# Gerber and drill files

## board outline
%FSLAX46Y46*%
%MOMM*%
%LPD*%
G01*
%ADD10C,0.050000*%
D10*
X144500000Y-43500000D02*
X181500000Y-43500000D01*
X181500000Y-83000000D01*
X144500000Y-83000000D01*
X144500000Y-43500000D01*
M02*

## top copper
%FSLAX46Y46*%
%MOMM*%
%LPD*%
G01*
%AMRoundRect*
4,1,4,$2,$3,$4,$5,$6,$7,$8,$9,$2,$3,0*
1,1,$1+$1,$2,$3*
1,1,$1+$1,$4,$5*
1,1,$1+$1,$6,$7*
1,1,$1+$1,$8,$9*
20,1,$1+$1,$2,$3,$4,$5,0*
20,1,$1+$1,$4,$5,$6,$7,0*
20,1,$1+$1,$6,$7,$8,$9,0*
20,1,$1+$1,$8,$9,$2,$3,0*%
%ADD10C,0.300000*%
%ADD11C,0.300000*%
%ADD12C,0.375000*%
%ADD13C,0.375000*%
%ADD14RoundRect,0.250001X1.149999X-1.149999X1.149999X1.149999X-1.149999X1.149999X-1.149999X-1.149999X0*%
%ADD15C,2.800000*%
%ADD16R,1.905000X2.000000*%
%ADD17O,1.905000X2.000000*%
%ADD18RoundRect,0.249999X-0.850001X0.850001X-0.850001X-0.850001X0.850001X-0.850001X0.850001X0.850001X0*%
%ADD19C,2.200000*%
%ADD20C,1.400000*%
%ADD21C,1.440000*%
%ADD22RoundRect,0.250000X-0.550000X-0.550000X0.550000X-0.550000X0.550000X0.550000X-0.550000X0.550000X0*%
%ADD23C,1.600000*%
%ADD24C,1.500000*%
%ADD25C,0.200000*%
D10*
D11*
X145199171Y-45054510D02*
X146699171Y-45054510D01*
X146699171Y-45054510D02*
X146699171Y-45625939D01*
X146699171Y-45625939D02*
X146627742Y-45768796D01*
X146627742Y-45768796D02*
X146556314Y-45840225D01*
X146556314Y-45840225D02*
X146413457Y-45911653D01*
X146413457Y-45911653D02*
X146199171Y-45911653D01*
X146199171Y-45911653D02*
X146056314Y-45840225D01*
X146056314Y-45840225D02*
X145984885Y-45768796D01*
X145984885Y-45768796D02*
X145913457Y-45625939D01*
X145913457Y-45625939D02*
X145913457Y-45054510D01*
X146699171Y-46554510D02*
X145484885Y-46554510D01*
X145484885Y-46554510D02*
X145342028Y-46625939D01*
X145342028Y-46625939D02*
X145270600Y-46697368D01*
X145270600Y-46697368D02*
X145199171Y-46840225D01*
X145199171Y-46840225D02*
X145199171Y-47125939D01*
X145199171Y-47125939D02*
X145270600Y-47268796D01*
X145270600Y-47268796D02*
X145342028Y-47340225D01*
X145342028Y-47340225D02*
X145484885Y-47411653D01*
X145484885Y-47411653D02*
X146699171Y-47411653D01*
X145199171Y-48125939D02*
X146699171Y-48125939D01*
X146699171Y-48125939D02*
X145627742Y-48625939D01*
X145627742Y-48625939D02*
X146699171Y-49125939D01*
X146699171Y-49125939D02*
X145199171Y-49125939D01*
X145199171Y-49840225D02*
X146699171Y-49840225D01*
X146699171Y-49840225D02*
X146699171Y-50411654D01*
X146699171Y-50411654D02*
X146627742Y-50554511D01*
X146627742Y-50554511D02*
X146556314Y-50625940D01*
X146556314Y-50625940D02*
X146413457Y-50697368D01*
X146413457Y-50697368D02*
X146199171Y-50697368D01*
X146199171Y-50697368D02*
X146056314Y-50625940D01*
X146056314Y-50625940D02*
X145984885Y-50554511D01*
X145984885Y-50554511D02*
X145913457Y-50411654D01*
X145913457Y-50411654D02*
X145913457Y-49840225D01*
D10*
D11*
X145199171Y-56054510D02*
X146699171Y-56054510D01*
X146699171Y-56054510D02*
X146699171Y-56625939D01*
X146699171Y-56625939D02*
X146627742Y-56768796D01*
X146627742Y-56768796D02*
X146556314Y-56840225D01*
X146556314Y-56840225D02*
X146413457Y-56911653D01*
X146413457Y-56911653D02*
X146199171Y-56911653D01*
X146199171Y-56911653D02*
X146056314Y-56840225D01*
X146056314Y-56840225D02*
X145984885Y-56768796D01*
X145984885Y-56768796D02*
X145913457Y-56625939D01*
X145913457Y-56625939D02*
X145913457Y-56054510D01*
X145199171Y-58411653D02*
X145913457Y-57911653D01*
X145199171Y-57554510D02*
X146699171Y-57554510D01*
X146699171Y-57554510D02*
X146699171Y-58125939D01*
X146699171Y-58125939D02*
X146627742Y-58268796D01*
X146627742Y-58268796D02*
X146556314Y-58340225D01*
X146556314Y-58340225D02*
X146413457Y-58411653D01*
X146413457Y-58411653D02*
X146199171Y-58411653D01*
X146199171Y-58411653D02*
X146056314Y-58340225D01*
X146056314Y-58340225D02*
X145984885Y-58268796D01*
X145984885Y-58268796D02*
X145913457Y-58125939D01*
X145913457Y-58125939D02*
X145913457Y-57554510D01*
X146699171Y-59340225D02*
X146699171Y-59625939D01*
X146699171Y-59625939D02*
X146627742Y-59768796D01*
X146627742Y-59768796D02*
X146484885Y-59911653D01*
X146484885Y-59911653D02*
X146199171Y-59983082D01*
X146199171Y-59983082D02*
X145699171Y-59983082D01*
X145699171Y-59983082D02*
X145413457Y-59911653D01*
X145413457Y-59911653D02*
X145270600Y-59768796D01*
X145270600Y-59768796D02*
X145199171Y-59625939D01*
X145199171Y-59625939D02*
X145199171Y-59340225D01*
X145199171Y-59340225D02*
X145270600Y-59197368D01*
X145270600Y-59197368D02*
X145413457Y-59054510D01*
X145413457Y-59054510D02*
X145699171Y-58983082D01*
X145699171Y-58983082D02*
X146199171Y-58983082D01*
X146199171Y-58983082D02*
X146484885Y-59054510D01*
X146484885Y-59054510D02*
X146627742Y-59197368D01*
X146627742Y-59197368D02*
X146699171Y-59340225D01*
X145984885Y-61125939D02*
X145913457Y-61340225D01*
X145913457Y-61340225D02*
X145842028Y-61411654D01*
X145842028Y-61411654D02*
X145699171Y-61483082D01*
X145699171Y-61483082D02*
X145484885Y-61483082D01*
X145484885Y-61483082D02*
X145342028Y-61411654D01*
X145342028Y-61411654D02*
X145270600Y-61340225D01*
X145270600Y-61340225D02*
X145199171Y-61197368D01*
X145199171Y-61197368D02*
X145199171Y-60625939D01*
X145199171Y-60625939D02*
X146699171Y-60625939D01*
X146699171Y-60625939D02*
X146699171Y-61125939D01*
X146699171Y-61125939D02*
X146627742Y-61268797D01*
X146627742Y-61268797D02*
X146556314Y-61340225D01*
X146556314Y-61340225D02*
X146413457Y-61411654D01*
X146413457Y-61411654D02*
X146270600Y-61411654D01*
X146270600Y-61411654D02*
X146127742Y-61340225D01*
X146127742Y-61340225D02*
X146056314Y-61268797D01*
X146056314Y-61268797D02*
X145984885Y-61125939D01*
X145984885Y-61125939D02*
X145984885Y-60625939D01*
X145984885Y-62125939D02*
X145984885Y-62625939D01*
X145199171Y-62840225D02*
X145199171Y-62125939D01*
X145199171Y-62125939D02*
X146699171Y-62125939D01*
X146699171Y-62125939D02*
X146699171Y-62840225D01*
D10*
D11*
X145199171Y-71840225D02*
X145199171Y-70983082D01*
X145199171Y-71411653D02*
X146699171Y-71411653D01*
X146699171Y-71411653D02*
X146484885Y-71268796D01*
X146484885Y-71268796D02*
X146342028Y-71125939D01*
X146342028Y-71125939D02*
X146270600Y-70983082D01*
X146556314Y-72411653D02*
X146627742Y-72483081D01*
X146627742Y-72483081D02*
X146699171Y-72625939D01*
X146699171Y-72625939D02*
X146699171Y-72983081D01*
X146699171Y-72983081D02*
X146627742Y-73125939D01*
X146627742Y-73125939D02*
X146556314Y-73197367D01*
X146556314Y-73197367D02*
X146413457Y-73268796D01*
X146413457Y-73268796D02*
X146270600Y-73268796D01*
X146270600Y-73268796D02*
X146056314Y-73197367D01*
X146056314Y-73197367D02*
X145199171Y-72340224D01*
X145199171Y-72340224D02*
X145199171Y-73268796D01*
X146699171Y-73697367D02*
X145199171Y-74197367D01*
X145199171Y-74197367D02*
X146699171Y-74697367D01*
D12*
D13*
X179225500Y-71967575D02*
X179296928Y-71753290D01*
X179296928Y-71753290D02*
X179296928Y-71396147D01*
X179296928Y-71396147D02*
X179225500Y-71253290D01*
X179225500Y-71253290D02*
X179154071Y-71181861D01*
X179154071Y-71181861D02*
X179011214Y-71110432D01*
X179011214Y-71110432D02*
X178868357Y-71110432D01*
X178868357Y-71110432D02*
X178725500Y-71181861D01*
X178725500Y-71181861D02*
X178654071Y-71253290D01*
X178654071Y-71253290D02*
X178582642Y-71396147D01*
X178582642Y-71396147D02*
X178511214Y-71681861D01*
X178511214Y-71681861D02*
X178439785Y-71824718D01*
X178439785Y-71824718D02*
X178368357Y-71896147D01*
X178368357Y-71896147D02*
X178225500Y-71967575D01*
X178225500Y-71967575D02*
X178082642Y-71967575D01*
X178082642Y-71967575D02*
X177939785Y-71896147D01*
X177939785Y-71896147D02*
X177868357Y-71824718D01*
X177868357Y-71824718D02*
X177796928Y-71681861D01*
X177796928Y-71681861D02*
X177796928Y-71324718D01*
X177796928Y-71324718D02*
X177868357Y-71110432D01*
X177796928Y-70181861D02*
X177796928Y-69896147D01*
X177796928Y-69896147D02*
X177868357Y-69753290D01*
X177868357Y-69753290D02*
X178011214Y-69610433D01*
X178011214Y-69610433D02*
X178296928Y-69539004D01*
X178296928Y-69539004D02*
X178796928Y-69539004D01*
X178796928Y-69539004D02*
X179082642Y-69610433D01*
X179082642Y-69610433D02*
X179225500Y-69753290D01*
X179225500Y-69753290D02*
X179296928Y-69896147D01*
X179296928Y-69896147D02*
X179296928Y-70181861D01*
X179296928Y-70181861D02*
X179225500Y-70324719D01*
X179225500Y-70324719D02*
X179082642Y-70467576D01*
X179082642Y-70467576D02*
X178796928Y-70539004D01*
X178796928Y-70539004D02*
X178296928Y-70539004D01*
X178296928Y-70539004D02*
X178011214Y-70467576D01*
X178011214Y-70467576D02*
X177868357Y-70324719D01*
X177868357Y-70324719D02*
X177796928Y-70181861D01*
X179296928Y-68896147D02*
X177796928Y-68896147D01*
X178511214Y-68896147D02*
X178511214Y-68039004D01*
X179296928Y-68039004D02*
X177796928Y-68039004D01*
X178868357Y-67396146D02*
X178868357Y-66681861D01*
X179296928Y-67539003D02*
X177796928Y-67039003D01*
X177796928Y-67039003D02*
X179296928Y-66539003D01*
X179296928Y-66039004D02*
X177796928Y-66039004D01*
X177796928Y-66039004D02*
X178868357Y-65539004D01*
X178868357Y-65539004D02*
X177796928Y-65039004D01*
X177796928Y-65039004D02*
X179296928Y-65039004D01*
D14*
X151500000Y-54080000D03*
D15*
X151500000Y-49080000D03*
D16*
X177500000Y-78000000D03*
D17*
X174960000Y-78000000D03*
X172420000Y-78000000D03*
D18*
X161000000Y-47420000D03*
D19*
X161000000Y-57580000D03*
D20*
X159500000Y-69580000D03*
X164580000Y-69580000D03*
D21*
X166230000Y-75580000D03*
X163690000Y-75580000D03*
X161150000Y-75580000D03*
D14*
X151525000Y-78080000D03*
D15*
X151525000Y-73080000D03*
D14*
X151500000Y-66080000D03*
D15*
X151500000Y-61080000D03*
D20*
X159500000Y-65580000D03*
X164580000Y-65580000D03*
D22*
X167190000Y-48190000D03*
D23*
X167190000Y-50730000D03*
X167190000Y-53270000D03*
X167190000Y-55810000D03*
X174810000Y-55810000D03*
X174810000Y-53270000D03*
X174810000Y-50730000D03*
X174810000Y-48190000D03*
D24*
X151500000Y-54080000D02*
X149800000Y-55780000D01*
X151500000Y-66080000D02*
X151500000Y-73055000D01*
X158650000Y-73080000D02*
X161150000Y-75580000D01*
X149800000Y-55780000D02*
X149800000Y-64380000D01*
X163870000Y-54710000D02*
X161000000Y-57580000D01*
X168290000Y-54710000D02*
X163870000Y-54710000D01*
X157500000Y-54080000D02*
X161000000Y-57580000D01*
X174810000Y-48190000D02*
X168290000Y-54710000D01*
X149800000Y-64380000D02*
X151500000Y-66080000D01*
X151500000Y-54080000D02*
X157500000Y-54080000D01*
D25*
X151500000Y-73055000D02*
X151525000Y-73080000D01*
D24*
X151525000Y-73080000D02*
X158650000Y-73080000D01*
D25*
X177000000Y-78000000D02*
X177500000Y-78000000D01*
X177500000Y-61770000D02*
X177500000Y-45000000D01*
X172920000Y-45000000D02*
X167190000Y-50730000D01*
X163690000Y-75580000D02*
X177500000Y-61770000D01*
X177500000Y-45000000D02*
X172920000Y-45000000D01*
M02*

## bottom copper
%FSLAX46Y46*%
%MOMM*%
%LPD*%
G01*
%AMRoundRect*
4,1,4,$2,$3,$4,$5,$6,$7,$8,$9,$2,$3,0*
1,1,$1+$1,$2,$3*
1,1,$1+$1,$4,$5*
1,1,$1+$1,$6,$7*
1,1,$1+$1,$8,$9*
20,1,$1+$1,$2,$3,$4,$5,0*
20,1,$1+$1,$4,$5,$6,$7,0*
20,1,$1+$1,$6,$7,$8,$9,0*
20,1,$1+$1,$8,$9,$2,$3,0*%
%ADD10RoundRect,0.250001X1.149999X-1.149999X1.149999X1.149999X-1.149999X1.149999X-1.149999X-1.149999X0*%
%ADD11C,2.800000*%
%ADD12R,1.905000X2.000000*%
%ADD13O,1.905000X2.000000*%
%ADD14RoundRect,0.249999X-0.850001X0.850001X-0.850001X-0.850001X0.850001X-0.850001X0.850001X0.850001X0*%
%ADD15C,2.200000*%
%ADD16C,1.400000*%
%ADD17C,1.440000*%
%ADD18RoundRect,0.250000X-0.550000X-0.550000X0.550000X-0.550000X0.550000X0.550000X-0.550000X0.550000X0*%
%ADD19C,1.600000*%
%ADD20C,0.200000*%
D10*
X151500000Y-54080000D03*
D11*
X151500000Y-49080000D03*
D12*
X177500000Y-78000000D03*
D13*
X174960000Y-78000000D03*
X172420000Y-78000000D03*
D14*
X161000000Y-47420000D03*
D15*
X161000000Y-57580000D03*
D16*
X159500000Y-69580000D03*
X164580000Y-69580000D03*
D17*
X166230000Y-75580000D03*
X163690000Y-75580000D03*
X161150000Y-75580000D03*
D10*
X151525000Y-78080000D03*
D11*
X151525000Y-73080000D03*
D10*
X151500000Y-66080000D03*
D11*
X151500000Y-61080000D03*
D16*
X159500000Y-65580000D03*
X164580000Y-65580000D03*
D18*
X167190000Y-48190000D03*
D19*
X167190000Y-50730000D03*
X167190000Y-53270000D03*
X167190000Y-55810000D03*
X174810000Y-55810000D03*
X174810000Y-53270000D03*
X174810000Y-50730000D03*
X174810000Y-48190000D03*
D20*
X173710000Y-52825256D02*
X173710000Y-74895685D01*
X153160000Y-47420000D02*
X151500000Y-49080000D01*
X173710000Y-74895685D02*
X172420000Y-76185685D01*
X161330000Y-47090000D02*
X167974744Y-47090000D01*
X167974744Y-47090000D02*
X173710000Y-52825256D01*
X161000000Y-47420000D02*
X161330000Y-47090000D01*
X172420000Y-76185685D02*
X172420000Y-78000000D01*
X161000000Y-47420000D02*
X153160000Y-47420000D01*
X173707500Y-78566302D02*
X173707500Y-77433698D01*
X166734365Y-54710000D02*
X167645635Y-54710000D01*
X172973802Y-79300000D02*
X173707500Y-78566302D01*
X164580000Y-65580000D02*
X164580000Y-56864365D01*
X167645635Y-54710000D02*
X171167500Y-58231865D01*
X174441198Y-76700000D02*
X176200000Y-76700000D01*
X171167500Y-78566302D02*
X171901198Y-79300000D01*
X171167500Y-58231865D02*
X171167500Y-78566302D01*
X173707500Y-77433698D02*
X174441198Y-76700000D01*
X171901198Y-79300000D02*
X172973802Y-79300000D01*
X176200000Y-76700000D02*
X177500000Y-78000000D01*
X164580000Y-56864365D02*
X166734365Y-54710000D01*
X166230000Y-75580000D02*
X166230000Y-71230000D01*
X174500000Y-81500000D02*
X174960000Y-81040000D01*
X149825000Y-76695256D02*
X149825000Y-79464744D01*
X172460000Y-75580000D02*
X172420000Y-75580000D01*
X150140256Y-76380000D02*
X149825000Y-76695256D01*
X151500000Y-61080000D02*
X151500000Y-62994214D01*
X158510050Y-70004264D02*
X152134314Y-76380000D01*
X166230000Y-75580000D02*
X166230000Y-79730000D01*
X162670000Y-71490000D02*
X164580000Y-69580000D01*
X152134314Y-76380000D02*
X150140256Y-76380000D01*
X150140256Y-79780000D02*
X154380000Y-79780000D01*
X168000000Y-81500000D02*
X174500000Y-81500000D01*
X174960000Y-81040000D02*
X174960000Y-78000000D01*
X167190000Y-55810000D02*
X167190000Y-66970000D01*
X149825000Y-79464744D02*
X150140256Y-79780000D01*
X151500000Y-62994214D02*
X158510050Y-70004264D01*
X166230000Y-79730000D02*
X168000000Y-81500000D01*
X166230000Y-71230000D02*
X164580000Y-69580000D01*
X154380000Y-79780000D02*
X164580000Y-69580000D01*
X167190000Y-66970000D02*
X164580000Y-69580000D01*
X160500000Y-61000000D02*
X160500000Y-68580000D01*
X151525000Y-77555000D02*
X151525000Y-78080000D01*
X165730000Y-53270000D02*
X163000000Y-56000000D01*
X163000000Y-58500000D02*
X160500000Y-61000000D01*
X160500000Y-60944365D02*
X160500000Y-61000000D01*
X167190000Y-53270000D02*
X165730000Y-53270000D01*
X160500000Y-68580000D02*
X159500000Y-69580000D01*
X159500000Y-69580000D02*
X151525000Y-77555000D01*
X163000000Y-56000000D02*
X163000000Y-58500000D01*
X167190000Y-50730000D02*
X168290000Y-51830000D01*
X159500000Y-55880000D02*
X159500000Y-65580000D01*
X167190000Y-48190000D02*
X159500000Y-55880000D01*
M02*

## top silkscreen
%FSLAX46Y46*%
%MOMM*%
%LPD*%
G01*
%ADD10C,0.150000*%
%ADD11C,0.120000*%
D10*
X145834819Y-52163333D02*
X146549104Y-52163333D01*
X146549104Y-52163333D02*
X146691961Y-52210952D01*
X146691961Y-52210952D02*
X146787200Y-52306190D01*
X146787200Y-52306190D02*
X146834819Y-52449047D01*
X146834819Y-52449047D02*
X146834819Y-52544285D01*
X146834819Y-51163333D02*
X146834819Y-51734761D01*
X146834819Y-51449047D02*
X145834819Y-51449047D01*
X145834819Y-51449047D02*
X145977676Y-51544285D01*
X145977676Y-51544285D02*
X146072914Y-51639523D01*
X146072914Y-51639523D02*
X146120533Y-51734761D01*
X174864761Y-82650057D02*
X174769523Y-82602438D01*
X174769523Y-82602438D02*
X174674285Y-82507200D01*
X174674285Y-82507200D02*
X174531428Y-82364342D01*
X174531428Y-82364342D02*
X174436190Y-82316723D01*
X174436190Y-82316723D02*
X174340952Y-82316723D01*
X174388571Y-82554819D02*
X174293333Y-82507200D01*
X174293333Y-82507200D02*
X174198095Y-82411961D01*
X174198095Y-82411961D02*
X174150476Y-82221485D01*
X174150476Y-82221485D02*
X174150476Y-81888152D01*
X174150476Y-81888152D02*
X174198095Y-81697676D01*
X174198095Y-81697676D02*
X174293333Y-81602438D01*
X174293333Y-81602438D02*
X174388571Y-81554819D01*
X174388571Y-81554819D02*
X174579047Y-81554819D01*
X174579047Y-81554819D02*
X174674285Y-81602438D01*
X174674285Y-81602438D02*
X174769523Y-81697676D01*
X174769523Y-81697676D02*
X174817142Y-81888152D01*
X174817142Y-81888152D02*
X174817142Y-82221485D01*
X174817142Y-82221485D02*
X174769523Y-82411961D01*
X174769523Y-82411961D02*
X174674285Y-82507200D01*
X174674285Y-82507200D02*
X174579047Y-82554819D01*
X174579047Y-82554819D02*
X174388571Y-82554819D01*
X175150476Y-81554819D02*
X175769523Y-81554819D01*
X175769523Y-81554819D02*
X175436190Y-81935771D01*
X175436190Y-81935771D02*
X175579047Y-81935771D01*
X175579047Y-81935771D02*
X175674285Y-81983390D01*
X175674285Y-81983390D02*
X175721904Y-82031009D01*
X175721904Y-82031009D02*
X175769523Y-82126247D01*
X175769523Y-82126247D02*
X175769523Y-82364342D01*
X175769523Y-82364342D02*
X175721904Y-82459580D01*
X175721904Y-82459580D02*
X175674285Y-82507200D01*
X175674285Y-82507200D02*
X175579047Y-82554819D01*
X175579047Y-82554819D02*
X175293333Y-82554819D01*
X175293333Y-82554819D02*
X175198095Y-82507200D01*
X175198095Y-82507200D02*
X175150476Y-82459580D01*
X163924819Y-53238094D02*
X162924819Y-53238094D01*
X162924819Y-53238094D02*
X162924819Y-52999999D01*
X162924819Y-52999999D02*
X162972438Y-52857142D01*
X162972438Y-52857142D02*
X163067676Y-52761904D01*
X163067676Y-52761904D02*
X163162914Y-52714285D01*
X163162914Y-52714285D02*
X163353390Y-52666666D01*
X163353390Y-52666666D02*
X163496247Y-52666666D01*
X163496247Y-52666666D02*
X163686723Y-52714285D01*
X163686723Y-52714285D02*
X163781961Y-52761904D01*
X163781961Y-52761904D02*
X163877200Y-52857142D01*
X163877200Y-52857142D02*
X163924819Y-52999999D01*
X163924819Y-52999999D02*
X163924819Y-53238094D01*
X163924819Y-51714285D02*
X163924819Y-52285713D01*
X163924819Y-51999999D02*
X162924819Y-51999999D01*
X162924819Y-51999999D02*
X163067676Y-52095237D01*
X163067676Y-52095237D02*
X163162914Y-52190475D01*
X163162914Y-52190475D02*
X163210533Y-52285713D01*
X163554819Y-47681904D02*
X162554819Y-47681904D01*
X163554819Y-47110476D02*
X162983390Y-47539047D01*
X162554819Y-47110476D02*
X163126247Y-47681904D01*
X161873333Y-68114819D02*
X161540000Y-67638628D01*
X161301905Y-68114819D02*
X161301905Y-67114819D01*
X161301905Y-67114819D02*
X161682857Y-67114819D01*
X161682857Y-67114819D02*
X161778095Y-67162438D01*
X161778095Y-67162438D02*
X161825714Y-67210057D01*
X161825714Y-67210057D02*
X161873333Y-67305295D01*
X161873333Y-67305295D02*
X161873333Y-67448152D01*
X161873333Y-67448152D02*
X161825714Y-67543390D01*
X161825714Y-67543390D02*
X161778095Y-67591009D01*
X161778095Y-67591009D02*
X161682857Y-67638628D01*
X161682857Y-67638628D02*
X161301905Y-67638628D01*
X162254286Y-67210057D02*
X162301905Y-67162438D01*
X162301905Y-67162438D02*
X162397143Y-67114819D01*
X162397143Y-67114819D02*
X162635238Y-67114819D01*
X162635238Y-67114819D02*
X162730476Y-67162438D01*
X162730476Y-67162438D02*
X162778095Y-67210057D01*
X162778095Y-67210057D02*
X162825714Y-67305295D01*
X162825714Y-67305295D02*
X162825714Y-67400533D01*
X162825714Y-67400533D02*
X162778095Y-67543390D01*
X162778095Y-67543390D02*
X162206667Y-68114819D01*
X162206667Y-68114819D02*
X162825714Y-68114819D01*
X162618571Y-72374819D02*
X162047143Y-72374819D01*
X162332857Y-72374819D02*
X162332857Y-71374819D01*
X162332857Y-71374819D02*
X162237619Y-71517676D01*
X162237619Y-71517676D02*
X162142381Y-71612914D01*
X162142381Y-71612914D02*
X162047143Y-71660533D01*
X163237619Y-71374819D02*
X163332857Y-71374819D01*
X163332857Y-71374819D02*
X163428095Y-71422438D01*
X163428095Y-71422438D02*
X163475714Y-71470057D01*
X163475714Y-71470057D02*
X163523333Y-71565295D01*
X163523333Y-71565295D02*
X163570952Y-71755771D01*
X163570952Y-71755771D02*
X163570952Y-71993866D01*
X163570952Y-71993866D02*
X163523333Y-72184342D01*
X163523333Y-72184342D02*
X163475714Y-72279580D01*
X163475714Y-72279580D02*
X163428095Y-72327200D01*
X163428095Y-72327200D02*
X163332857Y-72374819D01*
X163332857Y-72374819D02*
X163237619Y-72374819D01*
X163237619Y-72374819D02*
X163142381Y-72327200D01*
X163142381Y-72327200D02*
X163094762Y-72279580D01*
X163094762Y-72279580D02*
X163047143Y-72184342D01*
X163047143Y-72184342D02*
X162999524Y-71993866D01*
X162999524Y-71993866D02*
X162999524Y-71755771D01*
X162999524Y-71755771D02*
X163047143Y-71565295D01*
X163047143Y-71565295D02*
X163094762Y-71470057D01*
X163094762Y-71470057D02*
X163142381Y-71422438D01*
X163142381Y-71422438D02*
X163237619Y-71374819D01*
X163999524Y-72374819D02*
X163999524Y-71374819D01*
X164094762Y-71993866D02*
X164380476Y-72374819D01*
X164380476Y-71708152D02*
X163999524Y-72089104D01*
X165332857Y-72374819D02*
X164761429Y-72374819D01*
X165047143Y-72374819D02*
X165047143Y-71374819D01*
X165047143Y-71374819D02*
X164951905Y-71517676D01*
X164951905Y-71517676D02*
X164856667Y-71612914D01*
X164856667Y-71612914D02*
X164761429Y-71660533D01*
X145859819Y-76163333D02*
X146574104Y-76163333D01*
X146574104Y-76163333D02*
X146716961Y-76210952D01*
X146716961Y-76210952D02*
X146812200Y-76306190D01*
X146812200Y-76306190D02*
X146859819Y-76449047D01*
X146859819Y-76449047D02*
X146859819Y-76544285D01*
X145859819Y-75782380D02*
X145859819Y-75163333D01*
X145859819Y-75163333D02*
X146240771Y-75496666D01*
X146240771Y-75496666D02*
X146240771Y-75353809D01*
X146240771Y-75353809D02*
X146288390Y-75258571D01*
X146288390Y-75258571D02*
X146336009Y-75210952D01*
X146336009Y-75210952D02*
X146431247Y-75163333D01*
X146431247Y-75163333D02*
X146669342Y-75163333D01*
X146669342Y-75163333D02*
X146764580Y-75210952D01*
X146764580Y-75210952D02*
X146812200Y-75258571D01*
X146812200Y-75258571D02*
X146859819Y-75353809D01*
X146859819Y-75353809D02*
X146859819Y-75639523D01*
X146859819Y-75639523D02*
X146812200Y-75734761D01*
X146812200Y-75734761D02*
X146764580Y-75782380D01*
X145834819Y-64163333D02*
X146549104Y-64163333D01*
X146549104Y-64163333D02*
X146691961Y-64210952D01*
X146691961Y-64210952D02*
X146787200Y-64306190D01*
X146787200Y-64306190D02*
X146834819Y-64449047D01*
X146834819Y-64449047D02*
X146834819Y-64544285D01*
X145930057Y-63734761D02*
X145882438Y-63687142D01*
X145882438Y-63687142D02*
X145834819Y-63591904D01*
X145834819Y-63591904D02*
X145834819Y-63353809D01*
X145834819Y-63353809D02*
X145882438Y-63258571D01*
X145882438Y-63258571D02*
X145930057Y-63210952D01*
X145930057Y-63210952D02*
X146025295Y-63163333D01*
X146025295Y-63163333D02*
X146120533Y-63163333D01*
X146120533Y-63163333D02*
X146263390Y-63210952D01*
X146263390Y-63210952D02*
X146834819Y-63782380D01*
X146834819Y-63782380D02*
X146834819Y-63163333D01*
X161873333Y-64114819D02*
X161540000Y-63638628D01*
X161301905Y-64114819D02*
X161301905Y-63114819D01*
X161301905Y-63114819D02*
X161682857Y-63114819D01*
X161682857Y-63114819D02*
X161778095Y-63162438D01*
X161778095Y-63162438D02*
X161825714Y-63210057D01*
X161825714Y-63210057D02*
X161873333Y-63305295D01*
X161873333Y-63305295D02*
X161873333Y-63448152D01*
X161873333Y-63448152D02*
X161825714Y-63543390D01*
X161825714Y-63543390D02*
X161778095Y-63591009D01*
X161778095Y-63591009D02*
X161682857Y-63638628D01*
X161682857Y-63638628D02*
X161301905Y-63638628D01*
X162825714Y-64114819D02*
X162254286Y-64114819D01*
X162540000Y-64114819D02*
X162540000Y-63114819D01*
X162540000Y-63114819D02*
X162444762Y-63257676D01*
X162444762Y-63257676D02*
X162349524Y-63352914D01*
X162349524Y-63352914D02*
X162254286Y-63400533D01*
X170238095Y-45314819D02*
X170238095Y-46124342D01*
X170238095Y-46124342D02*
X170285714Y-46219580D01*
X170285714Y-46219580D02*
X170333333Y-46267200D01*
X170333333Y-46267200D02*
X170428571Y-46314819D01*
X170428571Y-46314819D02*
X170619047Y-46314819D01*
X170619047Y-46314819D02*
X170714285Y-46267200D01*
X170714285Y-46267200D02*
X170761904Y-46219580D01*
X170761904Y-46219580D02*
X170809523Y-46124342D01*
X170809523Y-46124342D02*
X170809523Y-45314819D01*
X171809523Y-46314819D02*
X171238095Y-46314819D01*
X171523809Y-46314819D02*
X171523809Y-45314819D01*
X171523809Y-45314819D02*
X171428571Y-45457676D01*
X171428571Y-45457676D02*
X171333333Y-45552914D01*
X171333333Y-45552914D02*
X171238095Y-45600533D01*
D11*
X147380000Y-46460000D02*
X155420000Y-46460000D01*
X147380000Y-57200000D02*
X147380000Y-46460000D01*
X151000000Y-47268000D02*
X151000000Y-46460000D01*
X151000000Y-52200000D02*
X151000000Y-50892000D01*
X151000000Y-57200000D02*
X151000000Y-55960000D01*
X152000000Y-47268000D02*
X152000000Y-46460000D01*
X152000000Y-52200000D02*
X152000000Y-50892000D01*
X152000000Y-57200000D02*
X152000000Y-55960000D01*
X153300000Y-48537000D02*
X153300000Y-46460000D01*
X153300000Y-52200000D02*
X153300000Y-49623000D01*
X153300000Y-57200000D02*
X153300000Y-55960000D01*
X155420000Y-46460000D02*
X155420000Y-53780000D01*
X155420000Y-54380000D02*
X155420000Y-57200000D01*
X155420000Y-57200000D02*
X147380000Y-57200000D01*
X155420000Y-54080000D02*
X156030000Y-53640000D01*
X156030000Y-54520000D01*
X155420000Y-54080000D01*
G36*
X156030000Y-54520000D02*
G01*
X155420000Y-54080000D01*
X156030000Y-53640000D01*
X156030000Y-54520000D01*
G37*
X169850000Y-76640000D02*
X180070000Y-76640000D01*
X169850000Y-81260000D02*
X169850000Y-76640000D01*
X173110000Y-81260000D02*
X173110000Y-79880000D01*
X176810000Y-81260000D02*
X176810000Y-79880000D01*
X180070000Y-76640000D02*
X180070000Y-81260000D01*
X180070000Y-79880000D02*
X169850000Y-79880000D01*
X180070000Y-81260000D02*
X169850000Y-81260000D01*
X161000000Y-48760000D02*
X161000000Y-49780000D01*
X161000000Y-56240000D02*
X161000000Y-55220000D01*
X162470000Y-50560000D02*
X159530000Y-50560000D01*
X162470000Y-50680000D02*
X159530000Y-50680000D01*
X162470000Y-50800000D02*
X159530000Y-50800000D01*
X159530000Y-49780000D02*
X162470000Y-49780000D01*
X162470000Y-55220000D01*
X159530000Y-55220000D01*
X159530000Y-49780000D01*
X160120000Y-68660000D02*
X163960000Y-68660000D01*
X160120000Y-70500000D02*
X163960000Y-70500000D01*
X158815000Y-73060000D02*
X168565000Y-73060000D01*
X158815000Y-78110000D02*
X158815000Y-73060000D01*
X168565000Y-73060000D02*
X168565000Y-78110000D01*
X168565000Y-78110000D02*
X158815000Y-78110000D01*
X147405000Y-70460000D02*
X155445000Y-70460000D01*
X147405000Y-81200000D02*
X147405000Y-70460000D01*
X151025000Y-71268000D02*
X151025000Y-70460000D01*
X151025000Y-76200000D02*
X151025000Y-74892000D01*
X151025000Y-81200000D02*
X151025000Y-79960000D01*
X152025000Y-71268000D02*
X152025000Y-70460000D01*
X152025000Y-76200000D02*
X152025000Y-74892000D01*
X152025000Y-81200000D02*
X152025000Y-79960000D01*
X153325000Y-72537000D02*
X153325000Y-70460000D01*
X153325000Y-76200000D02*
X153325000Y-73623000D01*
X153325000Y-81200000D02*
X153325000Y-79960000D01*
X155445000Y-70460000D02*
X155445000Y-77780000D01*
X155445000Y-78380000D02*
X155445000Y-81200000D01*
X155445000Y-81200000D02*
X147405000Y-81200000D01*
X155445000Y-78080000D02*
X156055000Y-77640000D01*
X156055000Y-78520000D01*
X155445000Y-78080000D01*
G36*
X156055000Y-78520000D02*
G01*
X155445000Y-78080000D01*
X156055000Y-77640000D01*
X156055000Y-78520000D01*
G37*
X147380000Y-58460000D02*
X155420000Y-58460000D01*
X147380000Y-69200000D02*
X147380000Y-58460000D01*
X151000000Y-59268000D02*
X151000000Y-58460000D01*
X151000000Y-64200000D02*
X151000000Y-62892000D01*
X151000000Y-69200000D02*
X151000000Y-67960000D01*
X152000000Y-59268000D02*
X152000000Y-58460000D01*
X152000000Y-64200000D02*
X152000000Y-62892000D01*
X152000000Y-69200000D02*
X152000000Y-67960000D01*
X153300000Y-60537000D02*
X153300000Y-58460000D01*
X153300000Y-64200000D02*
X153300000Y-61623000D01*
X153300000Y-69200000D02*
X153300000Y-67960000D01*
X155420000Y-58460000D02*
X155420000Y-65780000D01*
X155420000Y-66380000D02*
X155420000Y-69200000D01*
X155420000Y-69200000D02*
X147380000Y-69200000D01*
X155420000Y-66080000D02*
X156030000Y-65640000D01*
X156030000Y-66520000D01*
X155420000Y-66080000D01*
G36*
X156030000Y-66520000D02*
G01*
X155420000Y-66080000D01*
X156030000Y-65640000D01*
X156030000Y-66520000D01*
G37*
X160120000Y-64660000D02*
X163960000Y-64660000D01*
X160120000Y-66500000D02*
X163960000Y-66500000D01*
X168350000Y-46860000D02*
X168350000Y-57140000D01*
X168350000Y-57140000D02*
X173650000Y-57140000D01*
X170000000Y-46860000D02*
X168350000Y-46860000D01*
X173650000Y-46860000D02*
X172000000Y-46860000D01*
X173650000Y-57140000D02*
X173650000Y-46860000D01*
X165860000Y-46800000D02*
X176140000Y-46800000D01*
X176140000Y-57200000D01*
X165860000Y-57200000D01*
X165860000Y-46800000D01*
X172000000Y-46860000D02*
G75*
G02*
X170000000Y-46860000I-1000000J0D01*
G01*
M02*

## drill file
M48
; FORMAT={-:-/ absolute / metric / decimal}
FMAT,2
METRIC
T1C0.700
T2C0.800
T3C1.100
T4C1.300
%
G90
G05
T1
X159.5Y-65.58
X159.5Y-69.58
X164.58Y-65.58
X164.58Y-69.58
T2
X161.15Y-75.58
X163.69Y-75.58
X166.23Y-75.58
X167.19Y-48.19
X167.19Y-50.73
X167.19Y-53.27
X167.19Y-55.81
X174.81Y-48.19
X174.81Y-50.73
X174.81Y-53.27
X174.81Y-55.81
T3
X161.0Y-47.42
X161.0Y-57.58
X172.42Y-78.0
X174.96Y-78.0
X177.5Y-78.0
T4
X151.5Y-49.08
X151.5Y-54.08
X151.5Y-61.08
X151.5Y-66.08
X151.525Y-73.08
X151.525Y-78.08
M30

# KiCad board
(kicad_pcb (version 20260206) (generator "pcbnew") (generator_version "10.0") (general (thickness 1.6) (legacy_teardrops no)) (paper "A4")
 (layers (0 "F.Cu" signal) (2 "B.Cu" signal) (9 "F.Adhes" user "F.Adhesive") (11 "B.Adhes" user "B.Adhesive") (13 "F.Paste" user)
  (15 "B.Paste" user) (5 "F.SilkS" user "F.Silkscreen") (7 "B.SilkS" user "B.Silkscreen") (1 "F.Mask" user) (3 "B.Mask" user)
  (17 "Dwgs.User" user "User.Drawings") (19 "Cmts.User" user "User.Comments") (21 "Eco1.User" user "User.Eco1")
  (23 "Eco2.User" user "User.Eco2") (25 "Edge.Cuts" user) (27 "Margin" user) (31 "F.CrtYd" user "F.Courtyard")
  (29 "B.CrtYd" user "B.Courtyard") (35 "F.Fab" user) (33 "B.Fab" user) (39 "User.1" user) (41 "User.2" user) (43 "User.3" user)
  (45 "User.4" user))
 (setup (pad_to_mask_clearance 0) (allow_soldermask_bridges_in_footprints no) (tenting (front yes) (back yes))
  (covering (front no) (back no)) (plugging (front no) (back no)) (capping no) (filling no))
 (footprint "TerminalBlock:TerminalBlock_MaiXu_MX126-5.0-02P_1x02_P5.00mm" (layer "F.Cu") (at 151.5 54.08 90)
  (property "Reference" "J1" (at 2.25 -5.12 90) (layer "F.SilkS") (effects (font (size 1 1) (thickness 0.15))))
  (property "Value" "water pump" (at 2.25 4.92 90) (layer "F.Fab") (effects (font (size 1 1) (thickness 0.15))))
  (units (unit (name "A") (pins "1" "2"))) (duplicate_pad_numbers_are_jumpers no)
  (fp_line (start 7.62 -4.12) (end 7.62 3.92) (stroke (width 0.12) (type solid)) (layer "F.SilkS"))
  (fp_line (start -3.12 -4.12) (end 7.62 -4.12) (stroke (width 0.12) (type solid)) (layer "F.SilkS"))
  (fp_line (start 6.812 -0.5) (end 7.62 -0.5) (stroke (width 0.12) (type solid)) (layer "F.SilkS"))
  (fp_line (start 1.88 -0.5) (end 3.188 -0.5) (stroke (width 0.12) (type solid)) (layer "F.SilkS"))
  (fp_line (start -3.12 -0.5) (end -1.88 -0.5) (stroke (width 0.12) (type solid)) (layer "F.SilkS"))
  (fp_line (start 6.812 0.5) (end 7.62 0.5) (stroke (width 0.12) (type solid)) (layer "F.SilkS"))
  (fp_line (start 1.88 0.5) (end 3.188 0.5) (stroke (width 0.12) (type solid)) (layer "F.SilkS"))
  (fp_line (start -3.12 0.5) (end -1.88 0.5) (stroke (width 0.12) (type solid)) (layer "F.SilkS"))
  (fp_line (start 5.543 1.8) (end 7.62 1.8) (stroke (width 0.12) (type solid)) (layer "F.SilkS"))
  (fp_line (start 1.88 1.8) (end 4.457 1.8) (stroke (width 0.12) (type solid)) (layer "F.SilkS"))
  (fp_line (start -3.12 1.8) (end -1.88 1.8) (stroke (width 0.12) (type solid)) (layer "F.SilkS"))
  (fp_line (start 7.62 3.92) (end 0.3 3.92) (stroke (width 0.12) (type solid)) (layer "F.SilkS"))
  (fp_line (start -0.3 3.92) (end -3.12 3.92) (stroke (width 0.12) (type solid)) (layer "F.SilkS"))
  (fp_line (start -3.12 3.92) (end -3.12 -4.12) (stroke (width 0.12) (type solid)) (layer "F.SilkS"))
  (fp_poly (pts (xy 0 3.92) (xy 0.44 4.53) (xy -0.44 4.53)) (stroke (width 0.12) (type solid)) (fill yes) (layer "F.SilkS"))
  (pad "1" thru_hole roundrect (at 0 0 90) (size 2.8 2.8) (drill 1.3) (layers "*.Cu" "*.Mask") (remove_unused_layers no)
   (roundrect_rratio 0.089286) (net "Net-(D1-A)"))
  (pad "2" thru_hole circle (at 5 0 90) (size 2.8 2.8) (drill 1.3) (layers "*.Cu" "*.Mask") (remove_unused_layers no) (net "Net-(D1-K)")))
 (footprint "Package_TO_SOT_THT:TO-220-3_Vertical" (layer "F.Cu") (at 177.5 78 180)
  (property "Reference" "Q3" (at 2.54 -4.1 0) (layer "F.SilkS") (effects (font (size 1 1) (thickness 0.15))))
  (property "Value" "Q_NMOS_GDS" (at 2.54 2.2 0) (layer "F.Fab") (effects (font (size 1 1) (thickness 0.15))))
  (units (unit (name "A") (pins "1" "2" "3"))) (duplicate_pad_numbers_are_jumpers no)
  (fp_line (start 7.65 1.36) (end -2.57 1.36) (stroke (width 0.12) (type solid)) (layer "F.SilkS"))
  (fp_line (start 7.65 -3.26) (end 7.65 1.36) (stroke (width 0.12) (type solid)) (layer "F.SilkS"))
  (fp_line (start 4.39 -3.26) (end 4.39 -1.88) (stroke (width 0.12) (type solid)) (layer "F.SilkS"))
  (fp_line (start 0.69 -3.26) (end 0.69 -1.88) (stroke (width 0.12) (type solid)) (layer "F.SilkS"))
  (fp_line (start -2.57 1.36) (end -2.57 -3.26) (stroke (width 0.12) (type solid)) (layer "F.SilkS"))
  (fp_line (start -2.57 -1.88) (end 7.65 -1.88) (stroke (width 0.12) (type solid)) (layer "F.SilkS"))
  (fp_line (start -2.57 -3.26) (end 7.65 -3.26) (stroke (width 0.12) (type solid)) (layer "F.SilkS"))
  (pad "1" thru_hole rect (at 0 0 180) (size 1.905 2) (drill 1.1) (layers "*.Cu" "*.Mask") (remove_unused_layers no) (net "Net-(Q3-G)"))
  (pad "2" thru_hole oval (at 2.54 0 180) (size 1.905 2) (drill 1.1) (layers "*.Cu" "*.Mask") (remove_unused_layers no)
   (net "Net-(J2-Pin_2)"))
  (pad "3" thru_hole oval (at 5.08 0 180) (size 1.905 2) (drill 1.1) (layers "*.Cu" "*.Mask") (remove_unused_layers no) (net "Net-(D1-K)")))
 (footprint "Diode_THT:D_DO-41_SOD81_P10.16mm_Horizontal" (layer "F.Cu") (at 161 47.42 -90)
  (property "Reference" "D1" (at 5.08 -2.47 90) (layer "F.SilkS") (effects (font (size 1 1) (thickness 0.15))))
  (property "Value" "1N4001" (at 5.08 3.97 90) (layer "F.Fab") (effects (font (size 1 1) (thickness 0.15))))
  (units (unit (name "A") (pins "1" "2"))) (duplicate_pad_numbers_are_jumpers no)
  (fp_line (start 1.34 0) (end 2.36 0) (stroke (width 0.12) (type solid)) (layer "F.SilkS"))
  (fp_line (start 8.82 0) (end 7.8 0) (stroke (width 0.12) (type solid)) (layer "F.SilkS"))
  (fp_line (start 3.14 -1.47) (end 3.14 1.47) (stroke (width 0.12) (type solid)) (layer "F.SilkS"))
  (fp_line (start 3.26 -1.47) (end 3.26 1.47) (stroke (width 0.12) (type solid)) (layer "F.SilkS"))
  (fp_line (start 3.38 -1.47) (end 3.38 1.47) (stroke (width 0.12) (type solid)) (layer "F.SilkS"))
  (fp_rect (start 2.36 -1.47) (end 7.8 1.47) (stroke (width 0.12) (type solid)) (fill no) (layer "F.SilkS"))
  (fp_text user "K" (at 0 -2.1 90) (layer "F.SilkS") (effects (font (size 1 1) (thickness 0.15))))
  (pad "1" thru_hole roundrect (at 0 0 270) (size 2.2 2.2) (drill 1.1) (layers "*.Cu" "*.Mask") (remove_unused_layers no)
   (roundrect_rratio 0.113636) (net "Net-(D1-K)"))
  (pad "2" thru_hole circle (at 10.16 0 270) (size 2.2 2.2) (drill 1.1) (layers "*.Cu" "*.Mask") (remove_unused_layers no)
   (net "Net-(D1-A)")))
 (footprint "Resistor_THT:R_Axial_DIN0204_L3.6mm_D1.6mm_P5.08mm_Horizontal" (layer "F.Cu") (at 159.5 69.58)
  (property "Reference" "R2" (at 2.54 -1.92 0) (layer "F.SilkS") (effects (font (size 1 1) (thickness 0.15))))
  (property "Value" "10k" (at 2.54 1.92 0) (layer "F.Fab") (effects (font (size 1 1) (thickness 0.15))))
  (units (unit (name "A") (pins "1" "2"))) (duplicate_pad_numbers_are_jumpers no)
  (fp_line (start 0.62 -0.92) (end 4.46 -0.92) (stroke (width 0.12) (type solid)) (layer "F.SilkS"))
  (fp_line (start 0.62 0.92) (end 4.46 0.92) (stroke (width 0.12) (type solid)) (layer "F.SilkS"))
  (pad "1" thru_hole circle (at 0 0) (size 1.4 1.4) (drill 0.7) (layers "*.Cu" "*.Mask") (remove_unused_layers no) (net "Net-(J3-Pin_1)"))
  (pad "2" thru_hole circle (at 5.08 0) (size 1.4 1.4) (drill 0.7) (layers "*.Cu" "*.Mask") (remove_unused_layers no) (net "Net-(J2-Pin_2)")))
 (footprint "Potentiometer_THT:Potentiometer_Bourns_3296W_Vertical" (layer "F.Cu") (at 166.23 75.58)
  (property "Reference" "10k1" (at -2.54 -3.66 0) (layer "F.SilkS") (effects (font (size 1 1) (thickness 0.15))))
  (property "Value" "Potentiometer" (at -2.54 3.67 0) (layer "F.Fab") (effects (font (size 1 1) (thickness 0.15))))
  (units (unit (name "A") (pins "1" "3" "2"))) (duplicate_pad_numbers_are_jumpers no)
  (fp_line (start -7.415 -2.52) (end 2.335 -2.52) (stroke (width 0.12) (type solid)) (layer "F.SilkS"))
  (fp_line (start -7.415 2.53) (end -7.415 -2.52) (stroke (width 0.12) (type solid)) (layer "F.SilkS"))
  (fp_line (start 2.335 -2.52) (end 2.335 2.53) (stroke (width 0.12) (type solid)) (layer "F.SilkS"))
  (fp_line (start 2.335 2.53) (end -7.415 2.53) (stroke (width 0.12) (type solid)) (layer "F.SilkS"))
  (pad "1" thru_hole circle (at 0 0) (size 1.44 1.44) (drill 0.8) (layers "*.Cu" "*.Mask") (remove_unused_layers no) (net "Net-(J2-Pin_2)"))
  (pad "2" thru_hole circle (at -2.54 0) (size 1.44 1.44) (drill 0.8) (layers "*.Cu" "*.Mask") (remove_unused_layers no) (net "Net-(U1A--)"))
  (pad "3" thru_hole circle (at -5.08 0) (size 1.44 1.44) (drill 0.8) (layers "*.Cu" "*.Mask") (remove_unused_layers no) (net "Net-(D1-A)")))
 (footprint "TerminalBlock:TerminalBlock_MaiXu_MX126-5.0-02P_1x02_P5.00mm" (layer "F.Cu") (at 151.525 78.08 90)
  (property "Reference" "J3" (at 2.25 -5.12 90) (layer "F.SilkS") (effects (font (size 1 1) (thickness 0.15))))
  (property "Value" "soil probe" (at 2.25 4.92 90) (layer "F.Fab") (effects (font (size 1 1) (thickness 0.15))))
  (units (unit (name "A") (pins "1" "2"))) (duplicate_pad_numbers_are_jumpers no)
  (fp_line (start 7.62 -4.12) (end 7.62 3.92) (stroke (width 0.12) (type solid)) (layer "F.SilkS"))
  (fp_line (start -3.12 -4.12) (end 7.62 -4.12) (stroke (width 0.12) (type solid)) (layer "F.SilkS"))
  (fp_line (start 6.812 -0.5) (end 7.62 -0.5) (stroke (width 0.12) (type solid)) (layer "F.SilkS"))
  (fp_line (start 1.88 -0.5) (end 3.188 -0.5) (stroke (width 0.12) (type solid)) (layer "F.SilkS"))
  (fp_line (start -3.12 -0.5) (end -1.88 -0.5) (stroke (width 0.12) (type solid)) (layer "F.SilkS"))
  (fp_line (start 6.812 0.5) (end 7.62 0.5) (stroke (width 0.12) (type solid)) (layer "F.SilkS"))
  (fp_line (start 1.88 0.5) (end 3.188 0.5) (stroke (width 0.12) (type solid)) (layer "F.SilkS"))
  (fp_line (start -3.12 0.5) (end -1.88 0.5) (stroke (width 0.12) (type solid)) (layer "F.SilkS"))
  (fp_line (start 5.543 1.8) (end 7.62 1.8) (stroke (width 0.12) (type solid)) (layer "F.SilkS"))
  (fp_line (start 1.88 1.8) (end 4.457 1.8) (stroke (width 0.12) (type solid)) (layer "F.SilkS"))
  (fp_line (start -3.12 1.8) (end -1.88 1.8) (stroke (width 0.12) (type solid)) (layer "F.SilkS"))
  (fp_line (start 7.62 3.92) (end 0.3 3.92) (stroke (width 0.12) (type solid)) (layer "F.SilkS"))
  (fp_line (start -0.3 3.92) (end -3.12 3.92) (stroke (width 0.12) (type solid)) (layer "F.SilkS"))
  (fp_line (start -3.12 3.92) (end -3.12 -4.12) (stroke (width 0.12) (type solid)) (layer "F.SilkS"))
  (fp_poly (pts (xy 0 3.92) (xy 0.44 4.53) (xy -0.44 4.53)) (stroke (width 0.12) (type solid)) (fill yes) (layer "F.SilkS"))
  (pad "1" thru_hole roundrect (at 0 0 90) (size 2.8 2.8) (drill 1.3) (layers "*.Cu" "*.Mask") (remove_unused_layers no)
   (roundrect_rratio 0.089286) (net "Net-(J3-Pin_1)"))
  (pad "2" thru_hole circle (at 5 0 90) (size 2.8 2.8) (drill 1.3) (layers "*.Cu" "*.Mask") (remove_unused_layers no) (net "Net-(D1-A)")))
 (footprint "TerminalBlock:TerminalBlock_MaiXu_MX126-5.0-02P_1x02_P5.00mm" (layer "F.Cu") (at 151.5 66.08 90)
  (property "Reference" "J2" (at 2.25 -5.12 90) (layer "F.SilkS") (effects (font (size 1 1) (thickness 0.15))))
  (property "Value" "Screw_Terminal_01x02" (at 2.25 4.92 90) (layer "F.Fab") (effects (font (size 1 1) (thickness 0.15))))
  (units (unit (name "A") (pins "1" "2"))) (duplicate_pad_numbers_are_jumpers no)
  (fp_line (start 7.62 -4.12) (end 7.62 3.92) (stroke (width 0.12) (type solid)) (layer "F.SilkS"))
  (fp_line (start -3.12 -4.12) (end 7.62 -4.12) (stroke (width 0.12) (type solid)) (layer "F.SilkS"))
  (fp_line (start 6.812 -0.5) (end 7.62 -0.5) (stroke (width 0.12) (type solid)) (layer "F.SilkS"))
  (fp_line (start 1.88 -0.5) (end 3.188 -0.5) (stroke (width 0.12) (type solid)) (layer "F.SilkS"))
  (fp_line (start -3.12 -0.5) (end -1.88 -0.5) (stroke (width 0.12) (type solid)) (layer "F.SilkS"))
  (fp_line (start 6.812 0.5) (end 7.62 0.5) (stroke (width 0.12) (type solid)) (layer "F.SilkS"))
  (fp_line (start 1.88 0.5) (end 3.188 0.5) (stroke (width 0.12) (type solid)) (layer "F.SilkS"))
  (fp_line (start -3.12 0.5) (end -1.88 0.5) (stroke (width 0.12) (type solid)) (layer "F.SilkS"))
  (fp_line (start 5.543 1.8) (end 7.62 1.8) (stroke (width 0.12) (type solid)) (layer "F.SilkS"))
  (fp_line (start 1.88 1.8) (end 4.457 1.8) (stroke (width 0.12) (type solid)) (layer "F.SilkS"))
  (fp_line (start -3.12 1.8) (end -1.88 1.8) (stroke (width 0.12) (type solid)) (layer "F.SilkS"))
  (fp_line (start 7.62 3.92) (end 0.3 3.92) (stroke (width 0.12) (type solid)) (layer "F.SilkS"))
  (fp_line (start -0.3 3.92) (end -3.12 3.92) (stroke (width 0.12) (type solid)) (layer "F.SilkS"))
  (fp_line (start -3.12 3.92) (end -3.12 -4.12) (stroke (width 0.12) (type solid)) (layer "F.SilkS"))
  (fp_poly (pts (xy 0 3.92) (xy 0.44 4.53) (xy -0.44 4.53)) (stroke (width 0.12) (type solid)) (fill yes) (layer "F.SilkS"))
  (pad "1" thru_hole roundrect (at 0 0 90) (size 2.8 2.8) (drill 1.3) (layers "*.Cu" "*.Mask") (remove_unused_layers no)
   (roundrect_rratio 0.089286) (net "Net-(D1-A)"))
  (pad "2" thru_hole circle (at 5 0 90) (size 2.8 2.8) (drill 1.3) (layers "*.Cu" "*.Mask") (remove_unused_layers no) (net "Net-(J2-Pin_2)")))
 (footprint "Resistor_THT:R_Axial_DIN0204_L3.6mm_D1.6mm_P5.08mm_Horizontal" (layer "F.Cu") (at 159.5 65.58)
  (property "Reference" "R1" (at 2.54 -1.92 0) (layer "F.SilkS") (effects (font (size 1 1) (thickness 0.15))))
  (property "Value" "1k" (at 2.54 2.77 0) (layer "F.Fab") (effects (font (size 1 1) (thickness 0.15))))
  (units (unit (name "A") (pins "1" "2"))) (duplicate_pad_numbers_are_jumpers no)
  (fp_line (start 0.62 -0.92) (end 4.46 -0.92) (stroke (width 0.12) (type solid)) (layer "F.SilkS"))
  (fp_line (start 0.62 0.92) (end 4.46 0.92) (stroke (width 0.12) (type solid)) (layer "F.SilkS"))
  (pad "1" thru_hole circle (at 0 0) (size 1.4 1.4) (drill 0.7) (layers "*.Cu" "*.Mask") (remove_unused_layers no) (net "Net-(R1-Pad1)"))
  (pad "2" thru_hole circle (at 5.08 0) (size 1.4 1.4) (drill 0.7) (layers "*.Cu" "*.Mask") (remove_unused_layers no) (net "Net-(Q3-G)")))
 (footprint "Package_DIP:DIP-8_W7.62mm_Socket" (layer "F.Cu") (at 167.19 48.19)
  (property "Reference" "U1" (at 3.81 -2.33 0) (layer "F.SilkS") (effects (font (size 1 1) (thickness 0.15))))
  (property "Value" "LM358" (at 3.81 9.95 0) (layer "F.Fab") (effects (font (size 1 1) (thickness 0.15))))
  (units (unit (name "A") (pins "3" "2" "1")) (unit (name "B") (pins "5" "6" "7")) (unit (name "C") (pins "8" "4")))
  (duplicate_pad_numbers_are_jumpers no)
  (fp_line (start 1.16 -1.33) (end 1.16 8.95) (stroke (width 0.12) (type solid)) (layer "F.SilkS"))
  (fp_line (start 1.16 8.95) (end 6.46 8.95) (stroke (width 0.12) (type solid)) (layer "F.SilkS"))
  (fp_line (start 2.81 -1.33) (end 1.16 -1.33) (stroke (width 0.12) (type solid)) (layer "F.SilkS"))
  (fp_line (start 6.46 -1.33) (end 4.81 -1.33) (stroke (width 0.12) (type solid)) (layer "F.SilkS"))
  (fp_line (start 6.46 8.95) (end 6.46 -1.33) (stroke (width 0.12) (type solid)) (layer "F.SilkS"))
  (fp_rect (start -1.33 -1.39) (end 8.95 9.01) (stroke (width 0.12) (type solid)) (fill no) (layer "F.SilkS"))
  (fp_arc (start 4.81 -1.33) (mid 3.81 -0.33) (end 2.81 -1.33) (stroke (width 0.12) (type solid)) (layer "F.SilkS"))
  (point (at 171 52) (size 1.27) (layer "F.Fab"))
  (pad "1" thru_hole roundrect (at 0 0) (size 1.6 1.6) (drill 0.8) (layers "*.Cu" "*.Mask") (remove_unused_layers no)
   (roundrect_rratio 0.15625) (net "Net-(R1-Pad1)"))
  (pad "2" thru_hole circle (at 0 2.54) (size 1.6 1.6) (drill 0.8) (layers "*.Cu" "*.Mask") (remove_unused_layers no) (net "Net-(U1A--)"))
  (pad "3" thru_hole circle (at 0 5.08) (size 1.6 1.6) (drill 0.8) (layers "*.Cu" "*.Mask") (remove_unused_layers no) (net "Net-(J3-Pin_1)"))
  (pad "4" thru_hole circle (at 0 7.62) (size 1.6 1.6) (drill 0.8) (layers "*.Cu" "*.Mask") (remove_unused_layers no) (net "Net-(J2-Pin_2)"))
  (pad "5" thru_hole circle (at 7.62 7.62) (size 1.6 1.6) (drill 0.8) (layers "*.Cu" "*.Mask") (remove_unused_layers no))
  (pad "6" thru_hole circle (at 7.62 5.08) (size 1.6 1.6) (drill 0.8) (layers "*.Cu" "*.Mask") (remove_unused_layers no))
  (pad "7" thru_hole circle (at 7.62 2.54) (size 1.6 1.6) (drill 0.8) (layers "*.Cu" "*.Mask") (remove_unused_layers no))
  (pad "8" thru_hole circle (at 7.62 0) (size 1.6 1.6) (drill 0.8) (layers "*.Cu" "*.Mask") (remove_unused_layers no) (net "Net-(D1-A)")))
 (gr_rect (start 144.5 43.5) (end 181.5 83) (stroke (width 0.05) (type default)) (fill no) (layer "Edge.Cuts"))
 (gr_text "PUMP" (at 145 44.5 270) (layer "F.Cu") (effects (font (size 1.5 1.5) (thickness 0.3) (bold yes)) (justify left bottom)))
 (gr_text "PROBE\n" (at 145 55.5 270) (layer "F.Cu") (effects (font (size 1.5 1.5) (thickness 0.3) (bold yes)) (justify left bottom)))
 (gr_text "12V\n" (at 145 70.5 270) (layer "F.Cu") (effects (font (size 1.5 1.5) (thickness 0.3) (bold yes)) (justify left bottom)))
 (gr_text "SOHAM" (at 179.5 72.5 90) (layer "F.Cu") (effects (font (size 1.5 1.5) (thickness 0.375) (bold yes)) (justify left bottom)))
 (segment (start 151.5 54.08) (end 149.8 55.78) (width 1.5) (layer "F.Cu") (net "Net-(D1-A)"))
 (segment (start 151.5 66.08) (end 151.5 73.055) (width 1.5) (layer "F.Cu") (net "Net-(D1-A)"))
 (segment (start 158.65 73.08) (end 161.15 75.58) (width 1.5) (layer "F.Cu") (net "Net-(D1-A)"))
 (segment (start 149.8 55.78) (end 149.8 64.38) (width 1.5) (layer "F.Cu") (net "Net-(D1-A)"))
 (segment (start 163.87 54.71) (end 161 57.58) (width 1.5) (layer "F.Cu") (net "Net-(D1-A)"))
 (segment (start 168.29 54.71) (end 163.87 54.71) (width 1.5) (layer "F.Cu") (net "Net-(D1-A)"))
 (segment (start 157.5 54.08) (end 161 57.58) (width 1.5) (layer "F.Cu") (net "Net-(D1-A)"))
 (segment (start 174.81 48.19) (end 168.29 54.71) (width 1.5) (layer "F.Cu") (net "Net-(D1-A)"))
 (segment (start 149.8 64.38) (end 151.5 66.08) (width 1.5) (layer "F.Cu") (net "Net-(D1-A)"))
 (segment (start 151.5 54.08) (end 157.5 54.08) (width 1.5) (layer "F.Cu") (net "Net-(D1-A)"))
 (segment (start 151.5 73.055) (end 151.525 73.08) (width 0.2) (layer "F.Cu") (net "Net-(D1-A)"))
 (segment (start 151.525 73.08) (end 158.65 73.08) (width 1.5) (layer "F.Cu") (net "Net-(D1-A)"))
 (segment (start 173.71 52.825256) (end 173.71 74.895685) (width 0.2) (layer "B.Cu") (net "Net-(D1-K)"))
 (segment (start 153.16 47.42) (end 151.5 49.08) (width 0.2) (layer "B.Cu") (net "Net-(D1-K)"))
 (segment (start 173.71 74.895685) (end 172.42 76.185685) (width 0.2) (layer "B.Cu") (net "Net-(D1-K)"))
 (segment (start 161.33 47.09) (end 167.974744 47.09) (width 0.2) (layer "B.Cu") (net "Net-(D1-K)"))
 (segment (start 167.974744 47.09) (end 173.71 52.825256) (width 0.2) (layer "B.Cu") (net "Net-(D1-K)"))
 (segment (start 161 47.42) (end 161.33 47.09) (width 0.2) (layer "B.Cu") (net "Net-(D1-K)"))
 (segment (start 172.42 76.185685) (end 172.42 78) (width 0.2) (layer "B.Cu") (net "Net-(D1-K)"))
 (segment (start 161 47.42) (end 153.16 47.42) (width 0.2) (layer "B.Cu") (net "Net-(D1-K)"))
 (segment (start 177 78) (end 177.5 78) (width 0.2) (layer "F.Cu") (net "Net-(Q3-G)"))
 (segment (start 173.7075 78.566302) (end 173.7075 77.433698) (width 0.2) (layer "B.Cu") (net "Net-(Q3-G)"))
 (segment (start 166.734365 54.71) (end 167.645635 54.71) (width 0.2) (layer "B.Cu") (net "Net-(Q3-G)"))
 (segment (start 172.973802 79.3) (end 173.7075 78.566302) (width 0.2) (layer "B.Cu") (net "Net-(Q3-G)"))
 (segment (start 164.58 65.58) (end 164.58 56.864365) (width 0.2) (layer "B.Cu") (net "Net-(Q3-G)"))
 (segment (start 167.645635 54.71) (end 171.1675 58.231865) (width 0.2) (layer "B.Cu") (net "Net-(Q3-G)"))
 (segment (start 174.441198 76.7) (end 176.2 76.7) (width 0.2) (layer "B.Cu") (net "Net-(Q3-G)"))
 (segment (start 171.1675 78.566302) (end 171.901198 79.3) (width 0.2) (layer "B.Cu") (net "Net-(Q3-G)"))
 (segment (start 171.1675 58.231865) (end 171.1675 78.566302) (width 0.2) (layer "B.Cu") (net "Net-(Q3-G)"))
 (segment (start 173.7075 77.433698) (end 174.441198 76.7) (width 0.2) (layer "B.Cu") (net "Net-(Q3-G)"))
 (segment (start 171.901198 79.3) (end 172.973802 79.3) (width 0.2) (layer "B.Cu") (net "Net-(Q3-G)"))
 (segment (start 176.2 76.7) (end 177.5 78) (width 0.2) (layer "B.Cu") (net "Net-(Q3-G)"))
 (segment (start 164.58 56.864365) (end 166.734365 54.71) (width 0.2) (layer "B.Cu") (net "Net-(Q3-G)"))
 (segment (start 166.23 75.58) (end 166.23 71.23) (width 0.2) (layer "B.Cu") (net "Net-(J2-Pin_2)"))
 (segment (start 174.5 81.5) (end 174.96 81.04) (width 0.2) (layer "B.Cu") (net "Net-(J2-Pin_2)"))
 (segment (start 149.825 76.695256) (end 149.825 79.464744) (width 0.2) (layer "B.Cu") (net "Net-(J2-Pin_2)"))
 (segment (start 172.46 75.58) (end 172.42 75.58) (width 0.2) (layer "B.Cu") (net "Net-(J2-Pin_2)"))
 (segment (start 150.140256 76.38) (end 149.825 76.695256) (width 0.2) (layer "B.Cu") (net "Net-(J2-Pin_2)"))
 (segment (start 151.5 61.08) (end 151.5 62.994214) (width 0.2) (layer "B.Cu") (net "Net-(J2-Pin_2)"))
 (segment (start 158.51005 70.004264) (end 152.134314 76.38) (width 0.2) (layer "B.Cu") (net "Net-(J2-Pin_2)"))
 (segment (start 166.23 75.58) (end 166.23 79.73) (width 0.2) (layer "B.Cu") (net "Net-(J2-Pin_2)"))
 (segment (start 162.67 71.49) (end 164.58 69.58) (width 0.2) (layer "B.Cu") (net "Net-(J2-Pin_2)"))
 (segment (start 152.134314 76.38) (end 150.140256 76.38) (width 0.2) (layer "B.Cu") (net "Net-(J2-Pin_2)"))
 (segment (start 150.140256 79.78) (end 154.38 79.78) (width 0.2) (layer "B.Cu") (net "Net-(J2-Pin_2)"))
 (segment (start 168 81.5) (end 174.5 81.5) (width 0.2) (layer "B.Cu") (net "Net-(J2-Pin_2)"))
 (segment (start 174.96 81.04) (end 174.96 78) (width 0.2) (layer "B.Cu") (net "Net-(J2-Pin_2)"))
 (segment (start 167.19 55.81) (end 167.19 66.97) (width 0.2) (layer "B.Cu") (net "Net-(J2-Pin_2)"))
 (segment (start 149.825 79.464744) (end 150.140256 79.78) (width 0.2) (layer "B.Cu") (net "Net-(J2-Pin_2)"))
 (segment (start 151.5 62.994214) (end 158.51005 70.004264) (width 0.2) (layer "B.Cu") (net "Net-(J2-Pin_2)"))
 (segment (start 166.23 79.73) (end 168 81.5) (width 0.2) (layer "B.Cu") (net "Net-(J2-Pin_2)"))
 (segment (start 166.23 71.23) (end 164.58 69.58) (width 0.2) (layer "B.Cu") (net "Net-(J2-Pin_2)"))
 (segment (start 154.38 79.78) (end 164.58 69.58) (width 0.2) (layer "B.Cu") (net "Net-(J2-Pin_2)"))
 (segment (start 167.19 66.97) (end 164.58 69.58) (width 0.2) (layer "B.Cu") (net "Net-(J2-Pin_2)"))
 (segment (start 160.5 61) (end 160.5 68.58) (width 0.2) (layer "B.Cu") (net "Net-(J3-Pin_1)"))
 (segment (start 151.525 77.555) (end 151.525 78.08) (width 0.2) (layer "B.Cu") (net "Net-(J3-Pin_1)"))
 (segment (start 165.73 53.27) (end 163 56) (width 0.2) (layer "B.Cu") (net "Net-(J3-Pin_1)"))
 (segment (start 163 58.5) (end 160.5 61) (width 0.2) (layer "B.Cu") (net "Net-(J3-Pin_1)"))
 (segment (start 160.5 60.944365) (end 160.5 61) (width 0.2) (layer "B.Cu") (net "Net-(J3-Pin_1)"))
 (segment (start 167.19 53.27) (end 165.73 53.27) (width 0.2) (layer "B.Cu") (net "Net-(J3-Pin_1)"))
 (segment (start 160.5 68.58) (end 159.5 69.58) (width 0.2) (layer "B.Cu") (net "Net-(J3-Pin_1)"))
 (segment (start 159.5 69.58) (end 151.525 77.555) (width 0.2) (layer "B.Cu") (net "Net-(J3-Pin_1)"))
 (segment (start 163 56) (end 163 58.5) (width 0.2) (layer "B.Cu") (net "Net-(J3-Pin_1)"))
 (segment (start 177.5 61.77) (end 177.5 45) (width 0.2) (layer "F.Cu") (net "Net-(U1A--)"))
 (segment (start 172.92 45) (end 167.19 50.73) (width 0.2) (layer "F.Cu") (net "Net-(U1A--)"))
 (segment (start 163.69 75.58) (end 177.5 61.77) (width 0.2) (layer "F.Cu") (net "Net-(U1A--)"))
 (segment (start 177.5 45) (end 172.92 45) (width 0.2) (layer "F.Cu") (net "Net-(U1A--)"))
 (segment (start 167.19 50.73) (end 168.29 51.83) (width 0.2) (layer "B.Cu") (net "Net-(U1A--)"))
 (segment (start 159.5 55.88) (end 159.5 65.58) (width 0.2) (layer "B.Cu") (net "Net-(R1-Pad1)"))
 (segment (start 167.19 48.19) (end 159.5 55.88) (width 0.2) (layer "B.Cu") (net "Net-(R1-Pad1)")))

